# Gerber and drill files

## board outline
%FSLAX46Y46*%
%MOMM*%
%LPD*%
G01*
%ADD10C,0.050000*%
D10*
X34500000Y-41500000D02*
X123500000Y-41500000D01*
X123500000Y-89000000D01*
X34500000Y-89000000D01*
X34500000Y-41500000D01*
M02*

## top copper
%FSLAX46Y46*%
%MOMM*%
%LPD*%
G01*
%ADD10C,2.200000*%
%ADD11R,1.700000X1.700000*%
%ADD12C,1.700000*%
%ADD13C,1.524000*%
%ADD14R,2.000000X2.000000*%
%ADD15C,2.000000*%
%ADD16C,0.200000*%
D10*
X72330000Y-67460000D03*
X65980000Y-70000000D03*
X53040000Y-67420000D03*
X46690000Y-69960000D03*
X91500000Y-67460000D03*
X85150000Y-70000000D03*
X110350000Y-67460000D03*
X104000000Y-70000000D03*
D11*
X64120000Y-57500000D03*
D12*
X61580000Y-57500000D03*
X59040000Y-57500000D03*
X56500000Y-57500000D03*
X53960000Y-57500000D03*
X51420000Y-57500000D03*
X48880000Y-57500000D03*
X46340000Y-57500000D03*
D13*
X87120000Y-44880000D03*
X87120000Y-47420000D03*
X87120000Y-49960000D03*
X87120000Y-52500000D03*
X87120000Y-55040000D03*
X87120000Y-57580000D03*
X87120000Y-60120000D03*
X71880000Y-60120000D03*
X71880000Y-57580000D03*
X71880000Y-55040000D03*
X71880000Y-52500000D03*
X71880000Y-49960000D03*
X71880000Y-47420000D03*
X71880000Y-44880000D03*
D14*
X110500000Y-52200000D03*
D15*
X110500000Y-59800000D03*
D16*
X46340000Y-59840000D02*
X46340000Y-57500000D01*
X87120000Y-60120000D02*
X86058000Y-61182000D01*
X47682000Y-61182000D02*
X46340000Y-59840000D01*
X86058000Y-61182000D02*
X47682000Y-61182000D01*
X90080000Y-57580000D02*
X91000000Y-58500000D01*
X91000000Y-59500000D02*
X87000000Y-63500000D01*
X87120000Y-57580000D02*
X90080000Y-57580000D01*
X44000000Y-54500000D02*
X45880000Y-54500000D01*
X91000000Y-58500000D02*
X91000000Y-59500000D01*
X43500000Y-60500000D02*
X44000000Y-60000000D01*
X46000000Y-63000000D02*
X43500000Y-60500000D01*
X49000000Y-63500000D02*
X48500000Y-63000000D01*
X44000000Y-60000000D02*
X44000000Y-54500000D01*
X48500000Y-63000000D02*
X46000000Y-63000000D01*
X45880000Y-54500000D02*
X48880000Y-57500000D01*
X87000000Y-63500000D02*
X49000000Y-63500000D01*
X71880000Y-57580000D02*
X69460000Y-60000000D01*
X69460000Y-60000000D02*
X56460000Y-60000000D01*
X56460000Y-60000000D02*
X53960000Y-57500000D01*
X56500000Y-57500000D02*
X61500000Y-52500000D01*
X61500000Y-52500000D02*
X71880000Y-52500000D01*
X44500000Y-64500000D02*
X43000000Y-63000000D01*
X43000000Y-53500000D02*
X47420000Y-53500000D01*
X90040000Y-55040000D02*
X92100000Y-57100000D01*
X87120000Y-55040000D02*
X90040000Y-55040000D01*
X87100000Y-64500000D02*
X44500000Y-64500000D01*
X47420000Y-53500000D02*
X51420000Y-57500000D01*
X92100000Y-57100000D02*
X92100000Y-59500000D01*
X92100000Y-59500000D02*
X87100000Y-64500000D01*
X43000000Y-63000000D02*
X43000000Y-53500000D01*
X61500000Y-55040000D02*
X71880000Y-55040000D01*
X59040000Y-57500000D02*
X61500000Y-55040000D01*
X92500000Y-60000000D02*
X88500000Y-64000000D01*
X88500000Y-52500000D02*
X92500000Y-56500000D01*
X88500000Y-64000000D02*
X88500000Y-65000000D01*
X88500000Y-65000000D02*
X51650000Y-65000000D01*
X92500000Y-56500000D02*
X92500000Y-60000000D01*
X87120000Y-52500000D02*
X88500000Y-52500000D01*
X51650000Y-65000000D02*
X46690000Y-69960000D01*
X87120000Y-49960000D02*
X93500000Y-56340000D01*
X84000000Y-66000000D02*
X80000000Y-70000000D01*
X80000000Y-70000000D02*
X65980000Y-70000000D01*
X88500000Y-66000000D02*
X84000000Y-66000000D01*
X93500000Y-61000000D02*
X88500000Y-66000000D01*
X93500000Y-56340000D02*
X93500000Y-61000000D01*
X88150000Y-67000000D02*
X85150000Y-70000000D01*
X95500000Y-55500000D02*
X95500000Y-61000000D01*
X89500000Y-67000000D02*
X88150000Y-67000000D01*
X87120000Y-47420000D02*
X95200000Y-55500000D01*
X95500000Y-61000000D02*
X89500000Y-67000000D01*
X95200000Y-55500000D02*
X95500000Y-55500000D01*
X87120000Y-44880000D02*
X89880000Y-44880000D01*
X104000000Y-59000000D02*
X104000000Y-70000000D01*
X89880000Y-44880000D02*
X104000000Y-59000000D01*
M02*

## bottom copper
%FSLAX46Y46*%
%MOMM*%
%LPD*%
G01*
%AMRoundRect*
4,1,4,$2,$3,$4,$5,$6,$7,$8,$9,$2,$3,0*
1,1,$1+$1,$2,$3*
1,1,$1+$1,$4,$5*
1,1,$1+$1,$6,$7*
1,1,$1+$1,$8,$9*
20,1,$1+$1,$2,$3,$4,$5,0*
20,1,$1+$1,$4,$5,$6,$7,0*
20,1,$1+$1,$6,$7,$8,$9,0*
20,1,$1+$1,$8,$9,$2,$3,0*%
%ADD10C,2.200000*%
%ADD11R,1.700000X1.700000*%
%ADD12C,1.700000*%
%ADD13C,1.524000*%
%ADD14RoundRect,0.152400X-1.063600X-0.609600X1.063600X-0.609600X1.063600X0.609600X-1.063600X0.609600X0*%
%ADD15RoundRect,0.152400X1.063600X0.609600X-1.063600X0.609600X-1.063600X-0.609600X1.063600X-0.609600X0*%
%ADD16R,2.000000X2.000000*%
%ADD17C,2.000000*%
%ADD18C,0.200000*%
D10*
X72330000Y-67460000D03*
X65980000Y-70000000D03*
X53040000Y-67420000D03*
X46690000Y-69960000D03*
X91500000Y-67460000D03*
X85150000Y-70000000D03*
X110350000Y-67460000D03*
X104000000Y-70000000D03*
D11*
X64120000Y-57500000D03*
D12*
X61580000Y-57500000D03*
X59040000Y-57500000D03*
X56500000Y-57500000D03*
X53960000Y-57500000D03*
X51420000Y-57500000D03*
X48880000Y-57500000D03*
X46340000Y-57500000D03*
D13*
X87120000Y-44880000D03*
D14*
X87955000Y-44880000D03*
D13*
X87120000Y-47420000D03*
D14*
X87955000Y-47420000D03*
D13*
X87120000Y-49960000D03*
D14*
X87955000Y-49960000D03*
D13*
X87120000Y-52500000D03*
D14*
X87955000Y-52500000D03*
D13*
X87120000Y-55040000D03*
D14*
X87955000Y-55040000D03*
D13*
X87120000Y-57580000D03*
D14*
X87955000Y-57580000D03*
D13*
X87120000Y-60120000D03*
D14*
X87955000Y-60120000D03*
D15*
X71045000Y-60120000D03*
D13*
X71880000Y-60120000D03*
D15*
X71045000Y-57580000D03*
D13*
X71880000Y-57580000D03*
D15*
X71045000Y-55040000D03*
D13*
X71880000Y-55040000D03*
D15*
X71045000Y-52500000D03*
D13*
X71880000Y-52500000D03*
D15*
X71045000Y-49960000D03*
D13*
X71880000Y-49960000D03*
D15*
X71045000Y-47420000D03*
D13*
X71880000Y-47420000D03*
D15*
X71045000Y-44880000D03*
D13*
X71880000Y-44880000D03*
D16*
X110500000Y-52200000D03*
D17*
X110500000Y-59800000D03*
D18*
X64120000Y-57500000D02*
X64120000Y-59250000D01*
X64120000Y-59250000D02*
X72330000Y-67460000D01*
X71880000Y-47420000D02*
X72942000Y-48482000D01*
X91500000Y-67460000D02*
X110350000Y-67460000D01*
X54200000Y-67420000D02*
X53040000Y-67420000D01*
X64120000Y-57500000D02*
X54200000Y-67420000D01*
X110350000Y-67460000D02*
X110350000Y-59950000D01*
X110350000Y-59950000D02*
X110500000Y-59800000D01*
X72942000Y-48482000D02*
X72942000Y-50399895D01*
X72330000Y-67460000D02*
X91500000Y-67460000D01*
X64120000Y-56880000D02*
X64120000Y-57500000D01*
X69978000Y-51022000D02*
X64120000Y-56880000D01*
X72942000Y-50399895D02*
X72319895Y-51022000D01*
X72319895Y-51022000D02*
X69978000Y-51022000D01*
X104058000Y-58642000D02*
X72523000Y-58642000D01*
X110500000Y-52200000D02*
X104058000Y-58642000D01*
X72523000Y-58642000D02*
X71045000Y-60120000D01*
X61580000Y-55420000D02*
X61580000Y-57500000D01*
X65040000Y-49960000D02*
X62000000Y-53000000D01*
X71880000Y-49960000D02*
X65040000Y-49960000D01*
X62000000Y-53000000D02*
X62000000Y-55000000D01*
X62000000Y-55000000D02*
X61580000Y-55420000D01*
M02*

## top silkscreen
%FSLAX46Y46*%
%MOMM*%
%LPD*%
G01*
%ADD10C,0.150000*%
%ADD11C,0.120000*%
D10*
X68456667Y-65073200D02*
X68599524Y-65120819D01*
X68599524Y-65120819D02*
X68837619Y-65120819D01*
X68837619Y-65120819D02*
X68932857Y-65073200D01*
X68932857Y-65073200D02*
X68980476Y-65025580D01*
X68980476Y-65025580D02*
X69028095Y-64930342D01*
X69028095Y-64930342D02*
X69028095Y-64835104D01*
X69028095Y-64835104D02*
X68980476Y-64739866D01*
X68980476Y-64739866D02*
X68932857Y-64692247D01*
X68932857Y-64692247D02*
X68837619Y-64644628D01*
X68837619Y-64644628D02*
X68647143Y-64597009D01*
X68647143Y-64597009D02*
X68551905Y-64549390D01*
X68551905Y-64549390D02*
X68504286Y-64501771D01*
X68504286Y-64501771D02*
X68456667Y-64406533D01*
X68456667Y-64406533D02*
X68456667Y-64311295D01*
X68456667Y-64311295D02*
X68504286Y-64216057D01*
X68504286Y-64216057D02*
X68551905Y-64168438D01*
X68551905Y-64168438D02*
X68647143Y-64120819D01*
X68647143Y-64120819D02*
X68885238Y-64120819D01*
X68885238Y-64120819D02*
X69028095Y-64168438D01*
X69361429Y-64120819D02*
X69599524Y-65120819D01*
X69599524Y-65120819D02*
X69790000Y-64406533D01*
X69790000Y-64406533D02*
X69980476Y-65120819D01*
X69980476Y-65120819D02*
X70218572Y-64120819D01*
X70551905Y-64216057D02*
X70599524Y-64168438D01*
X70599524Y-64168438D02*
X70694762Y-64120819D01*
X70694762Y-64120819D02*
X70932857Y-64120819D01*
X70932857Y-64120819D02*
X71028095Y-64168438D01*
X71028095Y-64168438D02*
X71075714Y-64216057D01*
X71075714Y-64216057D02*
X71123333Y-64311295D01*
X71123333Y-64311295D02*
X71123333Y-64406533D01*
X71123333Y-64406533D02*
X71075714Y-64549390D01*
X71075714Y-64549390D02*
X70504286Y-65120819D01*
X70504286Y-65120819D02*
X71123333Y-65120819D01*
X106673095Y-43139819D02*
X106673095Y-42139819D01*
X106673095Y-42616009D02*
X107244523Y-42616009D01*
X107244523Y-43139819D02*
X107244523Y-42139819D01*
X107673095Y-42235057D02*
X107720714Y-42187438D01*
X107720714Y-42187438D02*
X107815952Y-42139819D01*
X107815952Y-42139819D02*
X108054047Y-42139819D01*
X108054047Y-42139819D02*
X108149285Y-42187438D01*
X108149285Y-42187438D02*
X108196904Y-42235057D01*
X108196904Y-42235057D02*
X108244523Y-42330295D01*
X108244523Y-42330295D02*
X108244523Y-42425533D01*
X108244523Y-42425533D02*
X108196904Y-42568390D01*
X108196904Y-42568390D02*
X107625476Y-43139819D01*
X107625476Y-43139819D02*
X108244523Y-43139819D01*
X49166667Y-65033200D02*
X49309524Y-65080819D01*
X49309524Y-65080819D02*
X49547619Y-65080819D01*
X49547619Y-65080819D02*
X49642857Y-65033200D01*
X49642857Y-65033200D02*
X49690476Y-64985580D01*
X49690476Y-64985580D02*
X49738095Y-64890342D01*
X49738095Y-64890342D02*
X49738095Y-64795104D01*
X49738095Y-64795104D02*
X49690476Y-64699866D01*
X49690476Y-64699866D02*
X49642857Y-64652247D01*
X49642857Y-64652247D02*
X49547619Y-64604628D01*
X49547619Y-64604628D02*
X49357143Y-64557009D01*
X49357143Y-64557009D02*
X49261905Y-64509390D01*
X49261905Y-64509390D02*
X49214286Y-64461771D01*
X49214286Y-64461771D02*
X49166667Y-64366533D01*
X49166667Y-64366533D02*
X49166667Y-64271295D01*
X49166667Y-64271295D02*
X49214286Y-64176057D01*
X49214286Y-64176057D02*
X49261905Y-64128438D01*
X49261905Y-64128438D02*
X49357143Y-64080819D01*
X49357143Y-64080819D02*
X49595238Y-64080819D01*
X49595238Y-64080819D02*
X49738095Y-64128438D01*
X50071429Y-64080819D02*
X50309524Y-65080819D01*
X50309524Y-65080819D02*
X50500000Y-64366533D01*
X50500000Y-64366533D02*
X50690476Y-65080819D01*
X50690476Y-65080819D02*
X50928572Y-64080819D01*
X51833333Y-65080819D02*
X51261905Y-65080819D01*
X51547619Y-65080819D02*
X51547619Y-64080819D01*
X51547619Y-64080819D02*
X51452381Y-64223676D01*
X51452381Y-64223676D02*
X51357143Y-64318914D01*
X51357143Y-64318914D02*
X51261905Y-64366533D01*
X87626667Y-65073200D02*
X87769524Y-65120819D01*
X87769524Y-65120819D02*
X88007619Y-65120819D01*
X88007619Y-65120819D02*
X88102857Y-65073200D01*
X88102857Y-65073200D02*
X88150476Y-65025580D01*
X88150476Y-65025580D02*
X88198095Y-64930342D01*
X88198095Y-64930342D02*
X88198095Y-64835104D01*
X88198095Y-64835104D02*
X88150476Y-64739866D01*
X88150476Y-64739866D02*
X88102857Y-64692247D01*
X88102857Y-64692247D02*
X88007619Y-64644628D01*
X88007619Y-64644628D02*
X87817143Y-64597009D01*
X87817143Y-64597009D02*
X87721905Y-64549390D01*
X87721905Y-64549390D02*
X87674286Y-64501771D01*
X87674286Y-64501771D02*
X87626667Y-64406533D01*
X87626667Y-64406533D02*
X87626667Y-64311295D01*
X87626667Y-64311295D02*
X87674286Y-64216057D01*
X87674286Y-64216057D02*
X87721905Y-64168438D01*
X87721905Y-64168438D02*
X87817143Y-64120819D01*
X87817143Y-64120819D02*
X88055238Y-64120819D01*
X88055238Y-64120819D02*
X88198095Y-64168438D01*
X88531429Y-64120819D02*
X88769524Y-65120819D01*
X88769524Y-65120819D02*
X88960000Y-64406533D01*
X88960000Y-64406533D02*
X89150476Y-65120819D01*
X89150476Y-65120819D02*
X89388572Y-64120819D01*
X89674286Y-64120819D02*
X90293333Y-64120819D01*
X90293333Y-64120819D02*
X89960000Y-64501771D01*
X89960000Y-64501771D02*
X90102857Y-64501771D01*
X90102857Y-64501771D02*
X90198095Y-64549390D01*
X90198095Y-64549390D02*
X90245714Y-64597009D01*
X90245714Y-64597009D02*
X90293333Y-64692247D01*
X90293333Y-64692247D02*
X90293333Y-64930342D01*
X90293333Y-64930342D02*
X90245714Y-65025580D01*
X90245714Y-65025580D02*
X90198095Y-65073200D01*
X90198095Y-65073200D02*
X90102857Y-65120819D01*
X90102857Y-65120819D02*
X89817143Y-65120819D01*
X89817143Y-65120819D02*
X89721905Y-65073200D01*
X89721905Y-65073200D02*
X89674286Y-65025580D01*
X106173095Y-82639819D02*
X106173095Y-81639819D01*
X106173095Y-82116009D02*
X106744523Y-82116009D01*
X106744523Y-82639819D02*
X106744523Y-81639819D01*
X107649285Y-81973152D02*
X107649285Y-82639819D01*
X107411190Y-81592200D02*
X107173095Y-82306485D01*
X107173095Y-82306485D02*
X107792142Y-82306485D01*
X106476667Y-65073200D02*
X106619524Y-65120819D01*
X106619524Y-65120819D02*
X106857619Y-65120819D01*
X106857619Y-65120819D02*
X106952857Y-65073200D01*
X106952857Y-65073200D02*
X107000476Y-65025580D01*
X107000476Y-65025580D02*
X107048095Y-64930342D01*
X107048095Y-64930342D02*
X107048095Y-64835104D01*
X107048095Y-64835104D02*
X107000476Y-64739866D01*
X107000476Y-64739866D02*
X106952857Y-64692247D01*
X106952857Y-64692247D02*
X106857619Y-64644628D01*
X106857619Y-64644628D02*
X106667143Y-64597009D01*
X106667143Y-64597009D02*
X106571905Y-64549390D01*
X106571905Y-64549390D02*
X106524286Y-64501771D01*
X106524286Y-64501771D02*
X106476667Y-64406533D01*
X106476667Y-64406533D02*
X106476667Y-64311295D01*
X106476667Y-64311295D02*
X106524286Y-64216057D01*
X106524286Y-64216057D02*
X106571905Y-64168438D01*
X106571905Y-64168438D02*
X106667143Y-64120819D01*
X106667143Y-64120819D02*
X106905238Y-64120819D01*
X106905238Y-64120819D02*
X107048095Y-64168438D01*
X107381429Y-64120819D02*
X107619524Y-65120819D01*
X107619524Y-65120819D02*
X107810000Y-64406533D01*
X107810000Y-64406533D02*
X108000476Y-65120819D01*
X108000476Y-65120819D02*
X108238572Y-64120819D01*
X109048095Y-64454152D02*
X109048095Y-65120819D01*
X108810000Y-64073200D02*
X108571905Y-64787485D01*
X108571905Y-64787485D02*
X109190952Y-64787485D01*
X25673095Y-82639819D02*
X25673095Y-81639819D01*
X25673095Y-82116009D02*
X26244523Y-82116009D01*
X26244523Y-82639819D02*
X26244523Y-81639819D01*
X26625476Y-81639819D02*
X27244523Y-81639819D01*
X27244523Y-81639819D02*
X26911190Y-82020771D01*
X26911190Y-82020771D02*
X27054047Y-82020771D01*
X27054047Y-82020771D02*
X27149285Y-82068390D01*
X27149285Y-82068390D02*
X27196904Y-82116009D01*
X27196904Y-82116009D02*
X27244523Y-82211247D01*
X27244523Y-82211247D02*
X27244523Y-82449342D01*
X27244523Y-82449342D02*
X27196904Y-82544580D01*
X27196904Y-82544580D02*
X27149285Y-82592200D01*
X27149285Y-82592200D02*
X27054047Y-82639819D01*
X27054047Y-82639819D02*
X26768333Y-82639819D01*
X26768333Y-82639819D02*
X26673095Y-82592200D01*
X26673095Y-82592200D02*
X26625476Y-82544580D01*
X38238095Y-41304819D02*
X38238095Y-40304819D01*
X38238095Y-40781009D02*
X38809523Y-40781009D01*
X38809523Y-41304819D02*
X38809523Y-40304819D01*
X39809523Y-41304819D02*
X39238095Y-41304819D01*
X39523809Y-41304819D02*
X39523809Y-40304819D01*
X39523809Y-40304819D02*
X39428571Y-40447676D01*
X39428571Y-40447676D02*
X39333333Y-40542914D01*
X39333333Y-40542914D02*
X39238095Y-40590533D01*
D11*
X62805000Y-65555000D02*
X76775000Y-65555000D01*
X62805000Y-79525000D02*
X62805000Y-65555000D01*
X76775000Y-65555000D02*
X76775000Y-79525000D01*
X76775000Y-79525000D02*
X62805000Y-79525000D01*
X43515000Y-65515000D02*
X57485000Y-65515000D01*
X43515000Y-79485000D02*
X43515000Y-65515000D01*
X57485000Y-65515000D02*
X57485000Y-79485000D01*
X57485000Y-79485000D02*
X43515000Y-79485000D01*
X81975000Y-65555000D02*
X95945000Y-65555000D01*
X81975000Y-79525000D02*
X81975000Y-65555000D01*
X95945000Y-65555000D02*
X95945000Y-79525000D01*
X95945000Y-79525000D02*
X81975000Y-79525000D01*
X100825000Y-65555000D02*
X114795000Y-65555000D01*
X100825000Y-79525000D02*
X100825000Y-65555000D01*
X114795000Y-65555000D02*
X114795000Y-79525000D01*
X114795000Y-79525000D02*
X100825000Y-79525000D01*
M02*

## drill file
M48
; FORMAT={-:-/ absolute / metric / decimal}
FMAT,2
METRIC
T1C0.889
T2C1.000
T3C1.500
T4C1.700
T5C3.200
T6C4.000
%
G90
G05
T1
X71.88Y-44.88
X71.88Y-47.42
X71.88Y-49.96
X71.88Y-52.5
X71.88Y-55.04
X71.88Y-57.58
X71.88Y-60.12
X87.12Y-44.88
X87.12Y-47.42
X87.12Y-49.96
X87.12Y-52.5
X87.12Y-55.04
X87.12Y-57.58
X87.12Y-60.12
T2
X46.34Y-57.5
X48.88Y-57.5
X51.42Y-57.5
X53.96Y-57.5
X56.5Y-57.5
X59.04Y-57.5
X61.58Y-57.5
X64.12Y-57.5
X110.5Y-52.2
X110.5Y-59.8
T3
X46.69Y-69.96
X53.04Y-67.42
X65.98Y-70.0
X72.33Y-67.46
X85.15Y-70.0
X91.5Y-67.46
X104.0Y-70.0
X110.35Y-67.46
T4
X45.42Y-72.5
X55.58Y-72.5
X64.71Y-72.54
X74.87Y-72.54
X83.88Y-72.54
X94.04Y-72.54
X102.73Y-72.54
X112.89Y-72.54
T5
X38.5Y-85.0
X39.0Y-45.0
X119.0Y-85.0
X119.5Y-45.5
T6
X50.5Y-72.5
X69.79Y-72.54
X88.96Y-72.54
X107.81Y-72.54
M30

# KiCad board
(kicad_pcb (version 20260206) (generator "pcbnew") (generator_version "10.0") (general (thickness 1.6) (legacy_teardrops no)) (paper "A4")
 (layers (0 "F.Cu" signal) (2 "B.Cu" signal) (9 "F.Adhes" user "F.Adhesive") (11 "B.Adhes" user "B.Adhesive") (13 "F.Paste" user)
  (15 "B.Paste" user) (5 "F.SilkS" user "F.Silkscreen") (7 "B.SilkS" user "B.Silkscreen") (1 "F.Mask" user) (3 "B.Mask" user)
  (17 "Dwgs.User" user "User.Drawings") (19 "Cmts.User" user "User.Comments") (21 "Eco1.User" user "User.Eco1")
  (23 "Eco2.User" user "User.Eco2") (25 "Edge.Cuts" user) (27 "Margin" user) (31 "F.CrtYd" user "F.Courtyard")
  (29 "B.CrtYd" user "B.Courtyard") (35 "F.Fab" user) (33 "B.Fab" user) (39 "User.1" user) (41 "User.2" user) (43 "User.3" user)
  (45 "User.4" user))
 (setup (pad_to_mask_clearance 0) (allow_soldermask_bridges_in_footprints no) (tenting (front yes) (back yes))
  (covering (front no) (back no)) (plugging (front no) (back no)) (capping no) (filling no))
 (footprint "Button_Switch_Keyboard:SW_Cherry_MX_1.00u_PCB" (layer "F.Cu") (at 72.33 67.46)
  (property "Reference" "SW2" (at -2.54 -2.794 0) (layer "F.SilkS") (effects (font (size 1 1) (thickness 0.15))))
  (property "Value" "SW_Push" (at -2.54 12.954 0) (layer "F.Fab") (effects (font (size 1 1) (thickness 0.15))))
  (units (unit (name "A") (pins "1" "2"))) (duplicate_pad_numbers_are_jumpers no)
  (fp_line (start -9.525 -1.905) (end 4.445 -1.905) (stroke (width 0.12) (type solid)) (layer "F.SilkS"))
  (fp_line (start -9.525 12.065) (end -9.525 -1.905) (stroke (width 0.12) (type solid)) (layer "F.SilkS"))
  (fp_line (start 4.445 -1.905) (end 4.445 12.065) (stroke (width 0.12) (type solid)) (layer "F.SilkS"))
  (fp_line (start 4.445 12.065) (end -9.525 12.065) (stroke (width 0.12) (type solid)) (layer "F.SilkS"))
  (pad "" np_thru_hole circle (at -7.62 5.08) (size 1.7 1.7) (drill 1.7) (layers "*.Cu" "*.Mask"))
  (pad "" np_thru_hole circle (at -2.54 5.08) (size 4 4) (drill 4) (layers "*.Cu" "*.Mask"))
  (pad "" np_thru_hole circle (at 2.54 5.08) (size 1.7 1.7) (drill 1.7) (layers "*.Cu" "*.Mask"))
  (pad "1" thru_hole circle (at 0 0) (size 2.2 2.2) (drill 1.5) (layers "*.Cu" "*.Mask") (remove_unused_layers no) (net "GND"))
  (pad "2" thru_hole circle (at -6.35 2.54) (size 2.2 2.2) (drill 1.5) (layers "*.Cu" "*.Mask") (remove_unused_layers no)
   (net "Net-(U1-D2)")))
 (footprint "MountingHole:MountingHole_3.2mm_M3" (layer "F.Cu") (at 119.5 45.5)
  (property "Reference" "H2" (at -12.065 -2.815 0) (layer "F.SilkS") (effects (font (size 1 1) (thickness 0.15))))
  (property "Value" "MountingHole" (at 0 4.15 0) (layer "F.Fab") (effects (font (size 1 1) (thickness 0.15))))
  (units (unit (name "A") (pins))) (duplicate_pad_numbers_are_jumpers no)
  (pad "" np_thru_hole circle (at 0 0) (size 3.2 3.2) (drill 3.2) (layers "*.Cu" "*.Mask")))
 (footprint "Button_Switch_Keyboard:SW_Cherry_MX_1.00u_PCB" (layer "F.Cu") (at 53.04 67.42)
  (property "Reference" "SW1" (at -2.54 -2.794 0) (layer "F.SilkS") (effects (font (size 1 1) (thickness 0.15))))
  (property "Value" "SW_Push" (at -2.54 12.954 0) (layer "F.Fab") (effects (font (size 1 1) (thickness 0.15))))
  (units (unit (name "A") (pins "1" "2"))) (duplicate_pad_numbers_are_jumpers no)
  (fp_line (start -9.525 -1.905) (end 4.445 -1.905) (stroke (width 0.12) (type solid)) (layer "F.SilkS"))
  (fp_line (start -9.525 12.065) (end -9.525 -1.905) (stroke (width 0.12) (type solid)) (layer "F.SilkS"))
  (fp_line (start 4.445 -1.905) (end 4.445 12.065) (stroke (width 0.12) (type solid)) (layer "F.SilkS"))
  (fp_line (start 4.445 12.065) (end -9.525 12.065) (stroke (width 0.12) (type solid)) (layer "F.SilkS"))
  (pad "" np_thru_hole circle (at -7.62 5.08) (size 1.7 1.7) (drill 1.7) (layers "*.Cu" "*.Mask"))
  (pad "" np_thru_hole circle (at -2.54 5.08) (size 4 4) (drill 4) (layers "*.Cu" "*.Mask"))
  (pad "" np_thru_hole circle (at 2.54 5.08) (size 1.7 1.7) (drill 1.7) (layers "*.Cu" "*.Mask"))
  (pad "1" thru_hole circle (at 0 0) (size 2.2 2.2) (drill 1.5) (layers "*.Cu" "*.Mask") (remove_unused_layers no) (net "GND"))
  (pad "2" thru_hole circle (at -6.35 2.54) (size 2.2 2.2) (drill 1.5) (layers "*.Cu" "*.Mask") (remove_unused_layers no)
   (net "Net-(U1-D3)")))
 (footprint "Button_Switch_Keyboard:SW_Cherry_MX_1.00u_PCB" (layer "F.Cu") (at 91.5 67.46)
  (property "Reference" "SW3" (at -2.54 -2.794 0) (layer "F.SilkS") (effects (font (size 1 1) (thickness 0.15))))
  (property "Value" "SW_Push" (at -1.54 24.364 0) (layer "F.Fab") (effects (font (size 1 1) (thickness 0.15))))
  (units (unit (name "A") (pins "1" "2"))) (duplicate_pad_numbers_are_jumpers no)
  (fp_line (start -9.525 -1.905) (end 4.445 -1.905) (stroke (width 0.12) (type solid)) (layer "F.SilkS"))
  (fp_line (start -9.525 12.065) (end -9.525 -1.905) (stroke (width 0.12) (type solid)) (layer "F.SilkS"))
  (fp_line (start 4.445 -1.905) (end 4.445 12.065) (stroke (width 0.12) (type solid)) (layer "F.SilkS"))
  (fp_line (start 4.445 12.065) (end -9.525 12.065) (stroke (width 0.12) (type solid)) (layer "F.SilkS"))
  (pad "" np_thru_hole circle (at -7.62 5.08) (size 1.7 1.7) (drill 1.7) (layers "*.Cu" "*.Mask"))
  (pad "" np_thru_hole circle (at -2.54 5.08) (size 4 4) (drill 4) (layers "*.Cu" "*.Mask"))
  (pad "" np_thru_hole circle (at 2.54 5.08) (size 1.7 1.7) (drill 1.7) (layers "*.Cu" "*.Mask"))
  (pad "1" thru_hole circle (at 0 0) (size 2.2 2.2) (drill 1.5) (layers "*.Cu" "*.Mask") (remove_unused_layers no) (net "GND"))
  (pad "2" thru_hole circle (at -6.35 2.54) (size 2.2 2.2) (drill 1.5) (layers "*.Cu" "*.Mask") (remove_unused_layers no)
   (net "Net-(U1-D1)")))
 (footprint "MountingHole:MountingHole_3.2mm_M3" (layer "F.Cu") (at 119 85)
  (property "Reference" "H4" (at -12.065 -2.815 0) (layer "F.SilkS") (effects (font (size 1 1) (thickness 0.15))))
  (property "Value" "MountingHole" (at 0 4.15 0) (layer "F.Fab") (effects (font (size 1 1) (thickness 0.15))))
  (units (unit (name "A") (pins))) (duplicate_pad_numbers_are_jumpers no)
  (pad "" np_thru_hole circle (at 0 0) (size 3.2 3.2) (drill 3.2) (layers "*.Cu" "*.Mask")))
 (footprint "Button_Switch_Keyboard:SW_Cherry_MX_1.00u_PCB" (layer "F.Cu") (at 110.35 67.46)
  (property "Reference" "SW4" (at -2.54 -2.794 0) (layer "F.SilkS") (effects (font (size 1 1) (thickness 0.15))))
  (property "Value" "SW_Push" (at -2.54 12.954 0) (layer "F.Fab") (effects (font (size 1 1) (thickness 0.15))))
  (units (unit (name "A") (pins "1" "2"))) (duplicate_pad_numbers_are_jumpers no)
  (fp_line (start -9.525 -1.905) (end 4.445 -1.905) (stroke (width 0.12) (type solid)) (layer "F.SilkS"))
  (fp_line (start -9.525 12.065) (end -9.525 -1.905) (stroke (width 0.12) (type solid)) (layer "F.SilkS"))
  (fp_line (start 4.445 -1.905) (end 4.445 12.065) (stroke (width 0.12) (type solid)) (layer "F.SilkS"))
  (fp_line (start 4.445 12.065) (end -9.525 12.065) (stroke (width 0.12) (type solid)) (layer "F.SilkS"))
  (pad "" np_thru_hole circle (at -7.62 5.08) (size 1.7 1.7) (drill 1.7) (layers "*.Cu" "*.Mask"))
  (pad "" np_thru_hole circle (at -2.54 5.08) (size 4 4) (drill 4) (layers "*.Cu" "*.Mask"))
  (pad "" np_thru_hole circle (at 2.54 5.08) (size 1.7 1.7) (drill 1.7) (layers "*.Cu" "*.Mask"))
  (pad "1" thru_hole circle (at 0 0) (size 2.2 2.2) (drill 1.5) (layers "*.Cu" "*.Mask") (remove_unused_layers no) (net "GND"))
  (pad "2" thru_hole circle (at -6.35 2.54) (size 2.2 2.2) (drill 1.5) (layers "*.Cu" "*.Mask") (remove_unused_layers no)
   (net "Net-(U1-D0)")))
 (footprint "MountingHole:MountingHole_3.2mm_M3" (layer "F.Cu") (at 38.5 85)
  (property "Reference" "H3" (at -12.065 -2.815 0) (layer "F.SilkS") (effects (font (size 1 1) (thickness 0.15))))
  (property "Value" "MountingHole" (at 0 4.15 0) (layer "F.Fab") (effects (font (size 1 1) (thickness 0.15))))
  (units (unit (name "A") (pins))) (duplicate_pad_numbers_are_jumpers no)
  (pad "" np_thru_hole circle (at 0 0) (size 3.2 3.2) (drill 3.2) (layers "*.Cu" "*.Mask")))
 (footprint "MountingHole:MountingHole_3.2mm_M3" (layer "F.Cu") (at 39 45)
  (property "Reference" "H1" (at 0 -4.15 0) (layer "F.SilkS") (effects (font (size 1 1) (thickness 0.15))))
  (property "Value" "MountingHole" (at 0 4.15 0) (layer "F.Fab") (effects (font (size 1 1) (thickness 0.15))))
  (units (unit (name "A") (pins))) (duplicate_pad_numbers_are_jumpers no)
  (pad "" np_thru_hole circle (at 0 0) (size 3.2 3.2) (drill 3.2) (layers "*.Cu" "*.Mask")))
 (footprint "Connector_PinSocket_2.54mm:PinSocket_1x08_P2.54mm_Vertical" (layer "B.Cu") (at 64.12 57.5 90)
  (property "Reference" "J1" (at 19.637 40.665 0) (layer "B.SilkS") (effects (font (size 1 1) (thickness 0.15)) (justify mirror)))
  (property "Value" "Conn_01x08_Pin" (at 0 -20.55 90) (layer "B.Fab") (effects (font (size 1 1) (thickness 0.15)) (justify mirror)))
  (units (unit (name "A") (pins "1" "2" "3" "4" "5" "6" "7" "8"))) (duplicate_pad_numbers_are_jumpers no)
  (pad "1" thru_hole rect (at 0 0 90) (size 1.7 1.7) (drill 1) (layers "*.Cu" "*.Mask") (remove_unused_layers no) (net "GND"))
  (pad "2" thru_hole circle (at 0 -2.54 90) (size 1.7 1.7) (drill 1) (layers "*.Cu" "*.Mask") (remove_unused_layers no) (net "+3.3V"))
  (pad "3" thru_hole circle (at 0 -5.08 90) (size 1.7 1.7) (drill 1) (layers "*.Cu" "*.Mask") (remove_unused_layers no) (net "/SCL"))
  (pad "4" thru_hole circle (at 0 -7.62 90) (size 1.7 1.7) (drill 1) (layers "*.Cu" "*.Mask") (remove_unused_layers no) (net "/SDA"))
  (pad "5" thru_hole circle (at 0 -10.16 90) (size 1.7 1.7) (drill 1) (layers "*.Cu" "*.Mask") (remove_unused_layers no) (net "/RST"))
  (pad "6" thru_hole circle (at 0 -12.7 90) (size 1.7 1.7) (drill 1) (layers "*.Cu" "*.Mask") (remove_unused_layers no) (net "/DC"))
  (pad "7" thru_hole circle (at 0 -15.24 90) (size 1.7 1.7) (drill 1) (layers "*.Cu" "*.Mask") (remove_unused_layers no) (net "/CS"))
  (pad "8" thru_hole circle (at 0 -17.78 90) (size 1.7 1.7) (drill 1) (layers "*.Cu" "*.Mask") (remove_unused_layers no) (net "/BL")))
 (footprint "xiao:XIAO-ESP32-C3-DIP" (layer "B.Cu") (at 79.5 52.5 90)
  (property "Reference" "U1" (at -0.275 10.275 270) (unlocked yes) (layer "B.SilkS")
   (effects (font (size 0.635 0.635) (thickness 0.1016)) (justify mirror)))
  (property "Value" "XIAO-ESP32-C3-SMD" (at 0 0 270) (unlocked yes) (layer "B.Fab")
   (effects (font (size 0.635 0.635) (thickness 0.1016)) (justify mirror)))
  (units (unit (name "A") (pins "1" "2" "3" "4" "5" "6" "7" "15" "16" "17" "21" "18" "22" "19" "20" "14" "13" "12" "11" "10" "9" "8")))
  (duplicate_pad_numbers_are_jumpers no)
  (pad "1" thru_hole circle (at 7.62 7.62) (size 1.524 1.524) (drill 0.889) (layers "*.Cu" "*.Mask") (remove_unused_layers no)
   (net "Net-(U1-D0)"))
  (pad "1" smd roundrect (at 7.62 8.455) (size 2.432 1.524) (layers "B.Cu" "B.Mask") (roundrect_rratio 0.1) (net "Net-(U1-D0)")
   (thermal_bridge_angle 45))
  (pad "2" thru_hole circle (at 5.08 7.62) (size 1.524 1.524) (drill 0.889) (layers "*.Cu" "*.Mask") (remove_unused_layers no)
   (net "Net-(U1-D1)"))
  (pad "2" smd roundrect (at 5.08 8.455) (size 2.432 1.524) (layers "B.Cu" "B.Mask") (roundrect_rratio 0.1) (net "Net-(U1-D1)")
   (thermal_bridge_angle 45))
  (pad "3" thru_hole circle (at 2.54 7.62) (size 1.524 1.524) (drill 0.889) (layers "*.Cu" "*.Mask") (remove_unused_layers no)
   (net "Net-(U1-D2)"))
  (pad "3" smd roundrect (at 2.54 8.455) (size 2.432 1.524) (layers "B.Cu" "B.Mask") (roundrect_rratio 0.1) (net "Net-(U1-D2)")
   (thermal_bridge_angle 45))
  (pad "4" thru_hole circle (at 0 7.62) (size 1.524 1.524) (drill 0.889) (layers "*.Cu" "*.Mask") (remove_unused_layers no)
   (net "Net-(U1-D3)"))
  (pad "4" smd roundrect (at 0 8.455) (size 2.432 1.524) (layers "B.Cu" "B.Mask") (roundrect_rratio 0.1) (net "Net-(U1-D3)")
   (thermal_bridge_angle 45))
  (pad "5" thru_hole circle (at -2.54 7.62) (size 1.524 1.524) (drill 0.889) (layers "*.Cu" "*.Mask") (remove_unused_layers no) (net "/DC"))
  (pad "5" smd roundrect (at -2.54 8.455) (size 2.432 1.524) (layers "B.Cu" "B.Mask") (roundrect_rratio 0.1) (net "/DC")
   (thermal_bridge_angle 45))
  (pad "6" thru_hole circle (at -5.08 7.62) (size 1.524 1.524) (drill 0.889) (layers "*.Cu" "*.Mask") (remove_unused_layers no) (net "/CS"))
  (pad "6" smd roundrect (at -5.08 8.455) (size 2.432 1.524) (layers "B.Cu" "B.Mask") (roundrect_rratio 0.1) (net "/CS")
   (thermal_bridge_angle 45))
  (pad "7" thru_hole circle (at -7.62 7.62) (size 1.524 1.524) (drill 0.889) (layers "*.Cu" "*.Mask") (remove_unused_layers no) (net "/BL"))
  (pad "7" smd roundrect (at -7.62 8.455) (size 2.432 1.524) (layers "B.Cu" "B.Mask") (roundrect_rratio 0.1) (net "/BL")
   (thermal_bridge_angle 45))
  (pad "8" smd roundrect (at -7.62 -8.455 180) (size 2.432 1.524) (layers "B.Cu" "B.Mask") (roundrect_rratio 0.1) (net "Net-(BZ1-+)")
   (thermal_bridge_angle 45))
  (pad "8" thru_hole circle (at -7.62 -7.62 180) (size 1.524 1.524) (drill 0.889) (layers "*.Cu" "*.Mask") (remove_unused_layers no)
   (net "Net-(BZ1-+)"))
  (pad "9" smd roundrect (at -5.08 -8.455 180) (size 2.432 1.524) (layers "B.Cu" "B.Mask") (roundrect_rratio 0.1) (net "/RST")
   (thermal_bridge_angle 45))
  (pad "9" thru_hole circle (at -5.08 -7.62 180) (size 1.524 1.524) (drill 0.889) (layers "*.Cu" "*.Mask") (remove_unused_layers no)
   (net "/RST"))
  (pad "10" smd roundrect (at -2.54 -8.455 180) (size 2.432 1.524) (layers "B.Cu" "B.Mask") (roundrect_rratio 0.1) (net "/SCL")
   (thermal_bridge_angle 45))
  (pad "10" thru_hole circle (at -2.54 -7.62 180) (size 1.524 1.524) (drill 0.889) (layers "*.Cu" "*.Mask") (remove_unused_layers no)
   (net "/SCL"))
  (pad "11" smd roundrect (at 0 -8.455 180) (size 2.432 1.524) (layers "B.Cu" "B.Mask") (roundrect_rratio 0.1) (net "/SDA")
   (thermal_bridge_angle 45))
  (pad "11" thru_hole circle (at 0 -7.62 180) (size 1.524 1.524) (drill 0.889) (layers "*.Cu" "*.Mask") (remove_unused_layers no)
   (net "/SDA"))
  (pad "12" smd roundrect (at 2.54 -8.455 180) (size 2.432 1.524) (layers "B.Cu" "B.Mask") (roundrect_rratio 0.1) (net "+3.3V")
   (thermal_bridge_angle 45))
  (pad "12" thru_hole circle (at 2.54 -7.62 180) (size 1.524 1.524) (drill 0.889) (layers "*.Cu" "*.Mask") (remove_unused_layers no)
   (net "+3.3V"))
  (pad "13" smd roundrect (at 5.08 -8.455 180) (size 2.432 1.524) (layers "B.Cu" "B.Mask") (roundrect_rratio 0.1) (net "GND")
   (thermal_bridge_angle 45))
  (pad "13" thru_hole circle (at 5.08 -7.62 180) (size 1.524 1.524) (drill 0.889) (layers "*.Cu" "*.Mask") (remove_unused_layers no)
   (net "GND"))
  (pad "14" smd roundrect (at 7.62 -8.455 180) (size 2.432 1.524) (layers "B.Cu" "B.Mask") (roundrect_rratio 0.1)
   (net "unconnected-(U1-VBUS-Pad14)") (thermal_bridge_angle 45))
  (pad "14" thru_hole circle (at 7.62 -7.62 180) (size 1.524 1.524) (drill 0.889) (layers "*.Cu" "*.Mask") (remove_unused_layers no)
   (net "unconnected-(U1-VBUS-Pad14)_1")))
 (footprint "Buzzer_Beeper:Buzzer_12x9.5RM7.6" (layer "B.Cu") (at 110.5 52.2 -90)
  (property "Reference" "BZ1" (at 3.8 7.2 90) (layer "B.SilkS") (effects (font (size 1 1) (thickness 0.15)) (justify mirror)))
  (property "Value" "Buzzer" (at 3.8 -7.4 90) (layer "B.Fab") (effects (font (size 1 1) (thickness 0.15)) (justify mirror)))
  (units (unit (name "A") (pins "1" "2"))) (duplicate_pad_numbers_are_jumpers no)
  (pad "1" thru_hole rect (at 0 0 270) (size 2 2) (drill 1) (layers "*.Cu" "*.Mask") (remove_unused_layers no) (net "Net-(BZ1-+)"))
  (pad "2" thru_hole circle (at 7.6 0 270) (size 2 2) (drill 1) (layers "*.Cu" "*.Mask") (remove_unused_layers no) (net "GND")))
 (gr_rect (start 34.5 41.5) (end 123.5 89) (stroke (width 0.05) (type default)) (fill no) (layer "Edge.Cuts"))
 (segment (start 64.12 57.5) (end 64.12 59.25) (width 0.2) (layer "B.Cu") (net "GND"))
 (segment (start 64.12 59.25) (end 72.33 67.46) (width 0.2) (layer "B.Cu") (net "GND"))
 (segment (start 71.88 47.42) (end 72.942 48.482) (width 0.2) (layer "B.Cu") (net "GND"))
 (segment (start 91.5 67.46) (end 110.35 67.46) (width 0.2) (layer "B.Cu") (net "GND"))
 (segment (start 54.2 67.42) (end 53.04 67.42) (width 0.2) (layer "B.Cu") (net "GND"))
 (segment (start 64.12 57.5) (end 54.2 67.42) (width 0.2) (layer "B.Cu") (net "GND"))
 (segment (start 110.35 67.46) (end 110.35 59.95) (width 0.2) (layer "B.Cu") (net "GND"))
 (segment (start 110.35 59.95) (end 110.5 59.8) (width 0.2) (layer "B.Cu") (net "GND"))
 (segment (start 72.942 48.482) (end 72.942 50.399895) (width 0.2) (layer "B.Cu") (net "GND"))
 (segment (start 72.33 67.46) (end 91.5 67.46) (width 0.2) (layer "B.Cu") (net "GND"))
 (segment (start 64.12 56.88) (end 64.12 57.5) (width 0.2) (layer "B.Cu") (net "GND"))
 (segment (start 69.978 51.022) (end 64.12 56.88) (width 0.2) (layer "B.Cu") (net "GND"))
 (segment (start 72.942 50.399895) (end 72.319895 51.022) (width 0.2) (layer "B.Cu") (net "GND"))
 (segment (start 72.319895 51.022) (end 69.978 51.022) (width 0.2) (layer "B.Cu") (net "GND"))
 (segment (start 104.058 58.642) (end 72.523 58.642) (width 0.2) (layer "B.Cu") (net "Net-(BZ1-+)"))
 (segment (start 110.5 52.2) (end 104.058 58.642) (width 0.2) (layer "B.Cu") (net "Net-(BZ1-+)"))
 (segment (start 72.523 58.642) (end 71.045 60.12) (width 0.2) (layer "B.Cu") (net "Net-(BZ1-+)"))
 (segment (start 46.34 59.84) (end 46.34 57.5) (width 0.2) (layer "F.Cu") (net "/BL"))
 (segment (start 87.12 60.12) (end 86.058 61.182) (width 0.2) (layer "F.Cu") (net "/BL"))
 (segment (start 47.682 61.182) (end 46.34 59.84) (width 0.2) (layer "F.Cu") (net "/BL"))
 (segment (start 86.058 61.182) (end 47.682 61.182) (width 0.2) (layer "F.Cu") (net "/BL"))
 (segment (start 61.58 55.42) (end 61.58 57.5) (width 0.2) (layer "B.Cu") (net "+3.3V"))
 (segment (start 65.04 49.96) (end 62 53) (width 0.2) (layer "B.Cu") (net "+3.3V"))
 (segment (start 71.88 49.96) (end 65.04 49.96) (width 0.2) (layer "B.Cu") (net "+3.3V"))
 (segment (start 62 53) (end 62 55) (width 0.2) (layer "B.Cu") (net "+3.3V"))
 (segment (start 62 55) (end 61.58 55.42) (width 0.2) (layer "B.Cu") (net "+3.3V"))
 (segment (start 90.08 57.58) (end 91 58.5) (width 0.2) (layer "F.Cu") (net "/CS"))
 (segment (start 91 59.5) (end 87 63.5) (width 0.2) (layer "F.Cu") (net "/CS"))
 (segment (start 87.12 57.58) (end 90.08 57.58) (width 0.2) (layer "F.Cu") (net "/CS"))
 (segment (start 44 54.5) (end 45.88 54.5) (width 0.2) (layer "F.Cu") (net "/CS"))
 (segment (start 91 58.5) (end 91 59.5) (width 0.2) (layer "F.Cu") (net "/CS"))
 (segment (start 43.5 60.5) (end 44 60) (width 0.2) (layer "F.Cu") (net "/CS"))
 (segment (start 46 63) (end 43.5 60.5) (width 0.2) (layer "F.Cu") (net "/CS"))
 (segment (start 49 63.5) (end 48.5 63) (width 0.2) (layer "F.Cu") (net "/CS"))
 (segment (start 44 60) (end 44 54.5) (width 0.2) (layer "F.Cu") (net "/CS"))
 (segment (start 48.5 63) (end 46 63) (width 0.2) (layer "F.Cu") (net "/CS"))
 (segment (start 45.88 54.5) (end 48.88 57.5) (width 0.2) (layer "F.Cu") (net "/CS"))
 (segment (start 87 63.5) (end 49 63.5) (width 0.2) (layer "F.Cu") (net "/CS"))
 (segment (start 71.88 57.58) (end 69.46 60) (width 0.2) (layer "F.Cu") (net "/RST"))
 (segment (start 69.46 60) (end 56.46 60) (width 0.2) (layer "F.Cu") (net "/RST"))
 (segment (start 56.46 60) (end 53.96 57.5) (width 0.2) (layer "F.Cu") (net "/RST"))
 (segment (start 56.5 57.5) (end 61.5 52.5) (width 0.2) (layer "F.Cu") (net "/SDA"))
 (segment (start 61.5 52.5) (end 71.88 52.5) (width 0.2) (layer "F.Cu") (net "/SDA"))
 (segment (start 44.5 64.5) (end 43 63) (width 0.2) (layer "F.Cu") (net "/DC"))
 (segment (start 43 53.5) (end 47.42 53.5) (width 0.2) (layer "F.Cu") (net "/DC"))
 (segment (start 90.04 55.04) (end 92.1 57.1) (width 0.2) (layer "F.Cu") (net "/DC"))
 (segment (start 87.12 55.04) (end 90.04 55.04) (width 0.2) (layer "F.Cu") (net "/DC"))
 (segment (start 87.1 64.5) (end 44.5 64.5) (width 0.2) (layer "F.Cu") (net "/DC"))
 (segment (start 47.42 53.5) (end 51.42 57.5) (width 0.2) (layer "F.Cu") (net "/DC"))
 (segment (start 92.1 57.1) (end 92.1 59.5) (width 0.2) (layer "F.Cu") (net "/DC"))
 (segment (start 92.1 59.5) (end 87.1 64.5) (width 0.2) (layer "F.Cu") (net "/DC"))
 (segment (start 43 63) (end 43 53.5) (width 0.2) (layer "F.Cu") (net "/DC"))
 (segment (start 61.5 55.04) (end 71.88 55.04) (width 0.2) (layer "F.Cu") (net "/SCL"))
 (segment (start 59.04 57.5) (end 61.5 55.04) (width 0.2) (layer "F.Cu") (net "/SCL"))
 (segment (start 92.5 60) (end 88.5 64) (width 0.2) (layer "F.Cu") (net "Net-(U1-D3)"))
 (segment (start 88.5 52.5) (end 92.5 56.5) (width 0.2) (layer "F.Cu") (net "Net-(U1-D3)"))
 (segment (start 88.5 64) (end 88.5 65) (width 0.2) (layer "F.Cu") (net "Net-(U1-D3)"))
 (segment (start 88.5 65) (end 51.65 65) (width 0.2) (layer "F.Cu") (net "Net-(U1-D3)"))
 (segment (start 92.5 56.5) (end 92.5 60) (width 0.2) (layer "F.Cu") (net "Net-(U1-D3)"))
 (segment (start 87.12 52.5) (end 88.5 52.5) (width 0.2) (layer "F.Cu") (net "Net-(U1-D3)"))
 (segment (start 51.65 65) (end 46.69 69.96) (width 0.2) (layer "F.Cu") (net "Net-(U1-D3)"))
 (segment (start 87.12 49.96) (end 93.5 56.34) (width 0.2) (layer "F.Cu") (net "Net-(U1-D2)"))
 (segment (start 84 66) (end 80 70) (width 0.2) (layer "F.Cu") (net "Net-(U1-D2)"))
 (segment (start 80 70) (end 65.98 70) (width 0.2) (layer "F.Cu") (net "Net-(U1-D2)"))
 (segment (start 88.5 66) (end 84 66) (width 0.2) (layer "F.Cu") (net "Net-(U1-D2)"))
 (segment (start 93.5 61) (end 88.5 66) (width 0.2) (layer "F.Cu") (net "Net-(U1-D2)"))
 (segment (start 93.5 56.34) (end 93.5 61) (width 0.2) (layer "F.Cu") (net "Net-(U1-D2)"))
 (segment (start 88.15 67) (end 85.15 70) (width 0.2) (layer "F.Cu") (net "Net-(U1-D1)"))
 (segment (start 95.5 55.5) (end 95.5 61) (width 0.2) (layer "F.Cu") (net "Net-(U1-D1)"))
 (segment (start 89.5 67) (end 88.15 67) (width 0.2) (layer "F.Cu") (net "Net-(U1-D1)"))
 (segment (start 87.12 47.42) (end 95.2 55.5) (width 0.2) (layer "F.Cu") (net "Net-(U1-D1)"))
 (segment (start 95.5 61) (end 89.5 67) (width 0.2) (layer "F.Cu") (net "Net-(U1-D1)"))
 (segment (start 95.2 55.5) (end 95.5 55.5) (width 0.2) (layer "F.Cu") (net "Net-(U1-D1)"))
 (segment (start 87.12 44.88) (end 89.88 44.88) (width 0.2) (layer "F.Cu") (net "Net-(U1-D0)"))
 (segment (start 104 59) (end 104 70) (width 0.2) (layer "F.Cu") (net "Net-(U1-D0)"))
 (segment (start 89.88 44.88) (end 104 59) (width 0.2) (layer "F.Cu") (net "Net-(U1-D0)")))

